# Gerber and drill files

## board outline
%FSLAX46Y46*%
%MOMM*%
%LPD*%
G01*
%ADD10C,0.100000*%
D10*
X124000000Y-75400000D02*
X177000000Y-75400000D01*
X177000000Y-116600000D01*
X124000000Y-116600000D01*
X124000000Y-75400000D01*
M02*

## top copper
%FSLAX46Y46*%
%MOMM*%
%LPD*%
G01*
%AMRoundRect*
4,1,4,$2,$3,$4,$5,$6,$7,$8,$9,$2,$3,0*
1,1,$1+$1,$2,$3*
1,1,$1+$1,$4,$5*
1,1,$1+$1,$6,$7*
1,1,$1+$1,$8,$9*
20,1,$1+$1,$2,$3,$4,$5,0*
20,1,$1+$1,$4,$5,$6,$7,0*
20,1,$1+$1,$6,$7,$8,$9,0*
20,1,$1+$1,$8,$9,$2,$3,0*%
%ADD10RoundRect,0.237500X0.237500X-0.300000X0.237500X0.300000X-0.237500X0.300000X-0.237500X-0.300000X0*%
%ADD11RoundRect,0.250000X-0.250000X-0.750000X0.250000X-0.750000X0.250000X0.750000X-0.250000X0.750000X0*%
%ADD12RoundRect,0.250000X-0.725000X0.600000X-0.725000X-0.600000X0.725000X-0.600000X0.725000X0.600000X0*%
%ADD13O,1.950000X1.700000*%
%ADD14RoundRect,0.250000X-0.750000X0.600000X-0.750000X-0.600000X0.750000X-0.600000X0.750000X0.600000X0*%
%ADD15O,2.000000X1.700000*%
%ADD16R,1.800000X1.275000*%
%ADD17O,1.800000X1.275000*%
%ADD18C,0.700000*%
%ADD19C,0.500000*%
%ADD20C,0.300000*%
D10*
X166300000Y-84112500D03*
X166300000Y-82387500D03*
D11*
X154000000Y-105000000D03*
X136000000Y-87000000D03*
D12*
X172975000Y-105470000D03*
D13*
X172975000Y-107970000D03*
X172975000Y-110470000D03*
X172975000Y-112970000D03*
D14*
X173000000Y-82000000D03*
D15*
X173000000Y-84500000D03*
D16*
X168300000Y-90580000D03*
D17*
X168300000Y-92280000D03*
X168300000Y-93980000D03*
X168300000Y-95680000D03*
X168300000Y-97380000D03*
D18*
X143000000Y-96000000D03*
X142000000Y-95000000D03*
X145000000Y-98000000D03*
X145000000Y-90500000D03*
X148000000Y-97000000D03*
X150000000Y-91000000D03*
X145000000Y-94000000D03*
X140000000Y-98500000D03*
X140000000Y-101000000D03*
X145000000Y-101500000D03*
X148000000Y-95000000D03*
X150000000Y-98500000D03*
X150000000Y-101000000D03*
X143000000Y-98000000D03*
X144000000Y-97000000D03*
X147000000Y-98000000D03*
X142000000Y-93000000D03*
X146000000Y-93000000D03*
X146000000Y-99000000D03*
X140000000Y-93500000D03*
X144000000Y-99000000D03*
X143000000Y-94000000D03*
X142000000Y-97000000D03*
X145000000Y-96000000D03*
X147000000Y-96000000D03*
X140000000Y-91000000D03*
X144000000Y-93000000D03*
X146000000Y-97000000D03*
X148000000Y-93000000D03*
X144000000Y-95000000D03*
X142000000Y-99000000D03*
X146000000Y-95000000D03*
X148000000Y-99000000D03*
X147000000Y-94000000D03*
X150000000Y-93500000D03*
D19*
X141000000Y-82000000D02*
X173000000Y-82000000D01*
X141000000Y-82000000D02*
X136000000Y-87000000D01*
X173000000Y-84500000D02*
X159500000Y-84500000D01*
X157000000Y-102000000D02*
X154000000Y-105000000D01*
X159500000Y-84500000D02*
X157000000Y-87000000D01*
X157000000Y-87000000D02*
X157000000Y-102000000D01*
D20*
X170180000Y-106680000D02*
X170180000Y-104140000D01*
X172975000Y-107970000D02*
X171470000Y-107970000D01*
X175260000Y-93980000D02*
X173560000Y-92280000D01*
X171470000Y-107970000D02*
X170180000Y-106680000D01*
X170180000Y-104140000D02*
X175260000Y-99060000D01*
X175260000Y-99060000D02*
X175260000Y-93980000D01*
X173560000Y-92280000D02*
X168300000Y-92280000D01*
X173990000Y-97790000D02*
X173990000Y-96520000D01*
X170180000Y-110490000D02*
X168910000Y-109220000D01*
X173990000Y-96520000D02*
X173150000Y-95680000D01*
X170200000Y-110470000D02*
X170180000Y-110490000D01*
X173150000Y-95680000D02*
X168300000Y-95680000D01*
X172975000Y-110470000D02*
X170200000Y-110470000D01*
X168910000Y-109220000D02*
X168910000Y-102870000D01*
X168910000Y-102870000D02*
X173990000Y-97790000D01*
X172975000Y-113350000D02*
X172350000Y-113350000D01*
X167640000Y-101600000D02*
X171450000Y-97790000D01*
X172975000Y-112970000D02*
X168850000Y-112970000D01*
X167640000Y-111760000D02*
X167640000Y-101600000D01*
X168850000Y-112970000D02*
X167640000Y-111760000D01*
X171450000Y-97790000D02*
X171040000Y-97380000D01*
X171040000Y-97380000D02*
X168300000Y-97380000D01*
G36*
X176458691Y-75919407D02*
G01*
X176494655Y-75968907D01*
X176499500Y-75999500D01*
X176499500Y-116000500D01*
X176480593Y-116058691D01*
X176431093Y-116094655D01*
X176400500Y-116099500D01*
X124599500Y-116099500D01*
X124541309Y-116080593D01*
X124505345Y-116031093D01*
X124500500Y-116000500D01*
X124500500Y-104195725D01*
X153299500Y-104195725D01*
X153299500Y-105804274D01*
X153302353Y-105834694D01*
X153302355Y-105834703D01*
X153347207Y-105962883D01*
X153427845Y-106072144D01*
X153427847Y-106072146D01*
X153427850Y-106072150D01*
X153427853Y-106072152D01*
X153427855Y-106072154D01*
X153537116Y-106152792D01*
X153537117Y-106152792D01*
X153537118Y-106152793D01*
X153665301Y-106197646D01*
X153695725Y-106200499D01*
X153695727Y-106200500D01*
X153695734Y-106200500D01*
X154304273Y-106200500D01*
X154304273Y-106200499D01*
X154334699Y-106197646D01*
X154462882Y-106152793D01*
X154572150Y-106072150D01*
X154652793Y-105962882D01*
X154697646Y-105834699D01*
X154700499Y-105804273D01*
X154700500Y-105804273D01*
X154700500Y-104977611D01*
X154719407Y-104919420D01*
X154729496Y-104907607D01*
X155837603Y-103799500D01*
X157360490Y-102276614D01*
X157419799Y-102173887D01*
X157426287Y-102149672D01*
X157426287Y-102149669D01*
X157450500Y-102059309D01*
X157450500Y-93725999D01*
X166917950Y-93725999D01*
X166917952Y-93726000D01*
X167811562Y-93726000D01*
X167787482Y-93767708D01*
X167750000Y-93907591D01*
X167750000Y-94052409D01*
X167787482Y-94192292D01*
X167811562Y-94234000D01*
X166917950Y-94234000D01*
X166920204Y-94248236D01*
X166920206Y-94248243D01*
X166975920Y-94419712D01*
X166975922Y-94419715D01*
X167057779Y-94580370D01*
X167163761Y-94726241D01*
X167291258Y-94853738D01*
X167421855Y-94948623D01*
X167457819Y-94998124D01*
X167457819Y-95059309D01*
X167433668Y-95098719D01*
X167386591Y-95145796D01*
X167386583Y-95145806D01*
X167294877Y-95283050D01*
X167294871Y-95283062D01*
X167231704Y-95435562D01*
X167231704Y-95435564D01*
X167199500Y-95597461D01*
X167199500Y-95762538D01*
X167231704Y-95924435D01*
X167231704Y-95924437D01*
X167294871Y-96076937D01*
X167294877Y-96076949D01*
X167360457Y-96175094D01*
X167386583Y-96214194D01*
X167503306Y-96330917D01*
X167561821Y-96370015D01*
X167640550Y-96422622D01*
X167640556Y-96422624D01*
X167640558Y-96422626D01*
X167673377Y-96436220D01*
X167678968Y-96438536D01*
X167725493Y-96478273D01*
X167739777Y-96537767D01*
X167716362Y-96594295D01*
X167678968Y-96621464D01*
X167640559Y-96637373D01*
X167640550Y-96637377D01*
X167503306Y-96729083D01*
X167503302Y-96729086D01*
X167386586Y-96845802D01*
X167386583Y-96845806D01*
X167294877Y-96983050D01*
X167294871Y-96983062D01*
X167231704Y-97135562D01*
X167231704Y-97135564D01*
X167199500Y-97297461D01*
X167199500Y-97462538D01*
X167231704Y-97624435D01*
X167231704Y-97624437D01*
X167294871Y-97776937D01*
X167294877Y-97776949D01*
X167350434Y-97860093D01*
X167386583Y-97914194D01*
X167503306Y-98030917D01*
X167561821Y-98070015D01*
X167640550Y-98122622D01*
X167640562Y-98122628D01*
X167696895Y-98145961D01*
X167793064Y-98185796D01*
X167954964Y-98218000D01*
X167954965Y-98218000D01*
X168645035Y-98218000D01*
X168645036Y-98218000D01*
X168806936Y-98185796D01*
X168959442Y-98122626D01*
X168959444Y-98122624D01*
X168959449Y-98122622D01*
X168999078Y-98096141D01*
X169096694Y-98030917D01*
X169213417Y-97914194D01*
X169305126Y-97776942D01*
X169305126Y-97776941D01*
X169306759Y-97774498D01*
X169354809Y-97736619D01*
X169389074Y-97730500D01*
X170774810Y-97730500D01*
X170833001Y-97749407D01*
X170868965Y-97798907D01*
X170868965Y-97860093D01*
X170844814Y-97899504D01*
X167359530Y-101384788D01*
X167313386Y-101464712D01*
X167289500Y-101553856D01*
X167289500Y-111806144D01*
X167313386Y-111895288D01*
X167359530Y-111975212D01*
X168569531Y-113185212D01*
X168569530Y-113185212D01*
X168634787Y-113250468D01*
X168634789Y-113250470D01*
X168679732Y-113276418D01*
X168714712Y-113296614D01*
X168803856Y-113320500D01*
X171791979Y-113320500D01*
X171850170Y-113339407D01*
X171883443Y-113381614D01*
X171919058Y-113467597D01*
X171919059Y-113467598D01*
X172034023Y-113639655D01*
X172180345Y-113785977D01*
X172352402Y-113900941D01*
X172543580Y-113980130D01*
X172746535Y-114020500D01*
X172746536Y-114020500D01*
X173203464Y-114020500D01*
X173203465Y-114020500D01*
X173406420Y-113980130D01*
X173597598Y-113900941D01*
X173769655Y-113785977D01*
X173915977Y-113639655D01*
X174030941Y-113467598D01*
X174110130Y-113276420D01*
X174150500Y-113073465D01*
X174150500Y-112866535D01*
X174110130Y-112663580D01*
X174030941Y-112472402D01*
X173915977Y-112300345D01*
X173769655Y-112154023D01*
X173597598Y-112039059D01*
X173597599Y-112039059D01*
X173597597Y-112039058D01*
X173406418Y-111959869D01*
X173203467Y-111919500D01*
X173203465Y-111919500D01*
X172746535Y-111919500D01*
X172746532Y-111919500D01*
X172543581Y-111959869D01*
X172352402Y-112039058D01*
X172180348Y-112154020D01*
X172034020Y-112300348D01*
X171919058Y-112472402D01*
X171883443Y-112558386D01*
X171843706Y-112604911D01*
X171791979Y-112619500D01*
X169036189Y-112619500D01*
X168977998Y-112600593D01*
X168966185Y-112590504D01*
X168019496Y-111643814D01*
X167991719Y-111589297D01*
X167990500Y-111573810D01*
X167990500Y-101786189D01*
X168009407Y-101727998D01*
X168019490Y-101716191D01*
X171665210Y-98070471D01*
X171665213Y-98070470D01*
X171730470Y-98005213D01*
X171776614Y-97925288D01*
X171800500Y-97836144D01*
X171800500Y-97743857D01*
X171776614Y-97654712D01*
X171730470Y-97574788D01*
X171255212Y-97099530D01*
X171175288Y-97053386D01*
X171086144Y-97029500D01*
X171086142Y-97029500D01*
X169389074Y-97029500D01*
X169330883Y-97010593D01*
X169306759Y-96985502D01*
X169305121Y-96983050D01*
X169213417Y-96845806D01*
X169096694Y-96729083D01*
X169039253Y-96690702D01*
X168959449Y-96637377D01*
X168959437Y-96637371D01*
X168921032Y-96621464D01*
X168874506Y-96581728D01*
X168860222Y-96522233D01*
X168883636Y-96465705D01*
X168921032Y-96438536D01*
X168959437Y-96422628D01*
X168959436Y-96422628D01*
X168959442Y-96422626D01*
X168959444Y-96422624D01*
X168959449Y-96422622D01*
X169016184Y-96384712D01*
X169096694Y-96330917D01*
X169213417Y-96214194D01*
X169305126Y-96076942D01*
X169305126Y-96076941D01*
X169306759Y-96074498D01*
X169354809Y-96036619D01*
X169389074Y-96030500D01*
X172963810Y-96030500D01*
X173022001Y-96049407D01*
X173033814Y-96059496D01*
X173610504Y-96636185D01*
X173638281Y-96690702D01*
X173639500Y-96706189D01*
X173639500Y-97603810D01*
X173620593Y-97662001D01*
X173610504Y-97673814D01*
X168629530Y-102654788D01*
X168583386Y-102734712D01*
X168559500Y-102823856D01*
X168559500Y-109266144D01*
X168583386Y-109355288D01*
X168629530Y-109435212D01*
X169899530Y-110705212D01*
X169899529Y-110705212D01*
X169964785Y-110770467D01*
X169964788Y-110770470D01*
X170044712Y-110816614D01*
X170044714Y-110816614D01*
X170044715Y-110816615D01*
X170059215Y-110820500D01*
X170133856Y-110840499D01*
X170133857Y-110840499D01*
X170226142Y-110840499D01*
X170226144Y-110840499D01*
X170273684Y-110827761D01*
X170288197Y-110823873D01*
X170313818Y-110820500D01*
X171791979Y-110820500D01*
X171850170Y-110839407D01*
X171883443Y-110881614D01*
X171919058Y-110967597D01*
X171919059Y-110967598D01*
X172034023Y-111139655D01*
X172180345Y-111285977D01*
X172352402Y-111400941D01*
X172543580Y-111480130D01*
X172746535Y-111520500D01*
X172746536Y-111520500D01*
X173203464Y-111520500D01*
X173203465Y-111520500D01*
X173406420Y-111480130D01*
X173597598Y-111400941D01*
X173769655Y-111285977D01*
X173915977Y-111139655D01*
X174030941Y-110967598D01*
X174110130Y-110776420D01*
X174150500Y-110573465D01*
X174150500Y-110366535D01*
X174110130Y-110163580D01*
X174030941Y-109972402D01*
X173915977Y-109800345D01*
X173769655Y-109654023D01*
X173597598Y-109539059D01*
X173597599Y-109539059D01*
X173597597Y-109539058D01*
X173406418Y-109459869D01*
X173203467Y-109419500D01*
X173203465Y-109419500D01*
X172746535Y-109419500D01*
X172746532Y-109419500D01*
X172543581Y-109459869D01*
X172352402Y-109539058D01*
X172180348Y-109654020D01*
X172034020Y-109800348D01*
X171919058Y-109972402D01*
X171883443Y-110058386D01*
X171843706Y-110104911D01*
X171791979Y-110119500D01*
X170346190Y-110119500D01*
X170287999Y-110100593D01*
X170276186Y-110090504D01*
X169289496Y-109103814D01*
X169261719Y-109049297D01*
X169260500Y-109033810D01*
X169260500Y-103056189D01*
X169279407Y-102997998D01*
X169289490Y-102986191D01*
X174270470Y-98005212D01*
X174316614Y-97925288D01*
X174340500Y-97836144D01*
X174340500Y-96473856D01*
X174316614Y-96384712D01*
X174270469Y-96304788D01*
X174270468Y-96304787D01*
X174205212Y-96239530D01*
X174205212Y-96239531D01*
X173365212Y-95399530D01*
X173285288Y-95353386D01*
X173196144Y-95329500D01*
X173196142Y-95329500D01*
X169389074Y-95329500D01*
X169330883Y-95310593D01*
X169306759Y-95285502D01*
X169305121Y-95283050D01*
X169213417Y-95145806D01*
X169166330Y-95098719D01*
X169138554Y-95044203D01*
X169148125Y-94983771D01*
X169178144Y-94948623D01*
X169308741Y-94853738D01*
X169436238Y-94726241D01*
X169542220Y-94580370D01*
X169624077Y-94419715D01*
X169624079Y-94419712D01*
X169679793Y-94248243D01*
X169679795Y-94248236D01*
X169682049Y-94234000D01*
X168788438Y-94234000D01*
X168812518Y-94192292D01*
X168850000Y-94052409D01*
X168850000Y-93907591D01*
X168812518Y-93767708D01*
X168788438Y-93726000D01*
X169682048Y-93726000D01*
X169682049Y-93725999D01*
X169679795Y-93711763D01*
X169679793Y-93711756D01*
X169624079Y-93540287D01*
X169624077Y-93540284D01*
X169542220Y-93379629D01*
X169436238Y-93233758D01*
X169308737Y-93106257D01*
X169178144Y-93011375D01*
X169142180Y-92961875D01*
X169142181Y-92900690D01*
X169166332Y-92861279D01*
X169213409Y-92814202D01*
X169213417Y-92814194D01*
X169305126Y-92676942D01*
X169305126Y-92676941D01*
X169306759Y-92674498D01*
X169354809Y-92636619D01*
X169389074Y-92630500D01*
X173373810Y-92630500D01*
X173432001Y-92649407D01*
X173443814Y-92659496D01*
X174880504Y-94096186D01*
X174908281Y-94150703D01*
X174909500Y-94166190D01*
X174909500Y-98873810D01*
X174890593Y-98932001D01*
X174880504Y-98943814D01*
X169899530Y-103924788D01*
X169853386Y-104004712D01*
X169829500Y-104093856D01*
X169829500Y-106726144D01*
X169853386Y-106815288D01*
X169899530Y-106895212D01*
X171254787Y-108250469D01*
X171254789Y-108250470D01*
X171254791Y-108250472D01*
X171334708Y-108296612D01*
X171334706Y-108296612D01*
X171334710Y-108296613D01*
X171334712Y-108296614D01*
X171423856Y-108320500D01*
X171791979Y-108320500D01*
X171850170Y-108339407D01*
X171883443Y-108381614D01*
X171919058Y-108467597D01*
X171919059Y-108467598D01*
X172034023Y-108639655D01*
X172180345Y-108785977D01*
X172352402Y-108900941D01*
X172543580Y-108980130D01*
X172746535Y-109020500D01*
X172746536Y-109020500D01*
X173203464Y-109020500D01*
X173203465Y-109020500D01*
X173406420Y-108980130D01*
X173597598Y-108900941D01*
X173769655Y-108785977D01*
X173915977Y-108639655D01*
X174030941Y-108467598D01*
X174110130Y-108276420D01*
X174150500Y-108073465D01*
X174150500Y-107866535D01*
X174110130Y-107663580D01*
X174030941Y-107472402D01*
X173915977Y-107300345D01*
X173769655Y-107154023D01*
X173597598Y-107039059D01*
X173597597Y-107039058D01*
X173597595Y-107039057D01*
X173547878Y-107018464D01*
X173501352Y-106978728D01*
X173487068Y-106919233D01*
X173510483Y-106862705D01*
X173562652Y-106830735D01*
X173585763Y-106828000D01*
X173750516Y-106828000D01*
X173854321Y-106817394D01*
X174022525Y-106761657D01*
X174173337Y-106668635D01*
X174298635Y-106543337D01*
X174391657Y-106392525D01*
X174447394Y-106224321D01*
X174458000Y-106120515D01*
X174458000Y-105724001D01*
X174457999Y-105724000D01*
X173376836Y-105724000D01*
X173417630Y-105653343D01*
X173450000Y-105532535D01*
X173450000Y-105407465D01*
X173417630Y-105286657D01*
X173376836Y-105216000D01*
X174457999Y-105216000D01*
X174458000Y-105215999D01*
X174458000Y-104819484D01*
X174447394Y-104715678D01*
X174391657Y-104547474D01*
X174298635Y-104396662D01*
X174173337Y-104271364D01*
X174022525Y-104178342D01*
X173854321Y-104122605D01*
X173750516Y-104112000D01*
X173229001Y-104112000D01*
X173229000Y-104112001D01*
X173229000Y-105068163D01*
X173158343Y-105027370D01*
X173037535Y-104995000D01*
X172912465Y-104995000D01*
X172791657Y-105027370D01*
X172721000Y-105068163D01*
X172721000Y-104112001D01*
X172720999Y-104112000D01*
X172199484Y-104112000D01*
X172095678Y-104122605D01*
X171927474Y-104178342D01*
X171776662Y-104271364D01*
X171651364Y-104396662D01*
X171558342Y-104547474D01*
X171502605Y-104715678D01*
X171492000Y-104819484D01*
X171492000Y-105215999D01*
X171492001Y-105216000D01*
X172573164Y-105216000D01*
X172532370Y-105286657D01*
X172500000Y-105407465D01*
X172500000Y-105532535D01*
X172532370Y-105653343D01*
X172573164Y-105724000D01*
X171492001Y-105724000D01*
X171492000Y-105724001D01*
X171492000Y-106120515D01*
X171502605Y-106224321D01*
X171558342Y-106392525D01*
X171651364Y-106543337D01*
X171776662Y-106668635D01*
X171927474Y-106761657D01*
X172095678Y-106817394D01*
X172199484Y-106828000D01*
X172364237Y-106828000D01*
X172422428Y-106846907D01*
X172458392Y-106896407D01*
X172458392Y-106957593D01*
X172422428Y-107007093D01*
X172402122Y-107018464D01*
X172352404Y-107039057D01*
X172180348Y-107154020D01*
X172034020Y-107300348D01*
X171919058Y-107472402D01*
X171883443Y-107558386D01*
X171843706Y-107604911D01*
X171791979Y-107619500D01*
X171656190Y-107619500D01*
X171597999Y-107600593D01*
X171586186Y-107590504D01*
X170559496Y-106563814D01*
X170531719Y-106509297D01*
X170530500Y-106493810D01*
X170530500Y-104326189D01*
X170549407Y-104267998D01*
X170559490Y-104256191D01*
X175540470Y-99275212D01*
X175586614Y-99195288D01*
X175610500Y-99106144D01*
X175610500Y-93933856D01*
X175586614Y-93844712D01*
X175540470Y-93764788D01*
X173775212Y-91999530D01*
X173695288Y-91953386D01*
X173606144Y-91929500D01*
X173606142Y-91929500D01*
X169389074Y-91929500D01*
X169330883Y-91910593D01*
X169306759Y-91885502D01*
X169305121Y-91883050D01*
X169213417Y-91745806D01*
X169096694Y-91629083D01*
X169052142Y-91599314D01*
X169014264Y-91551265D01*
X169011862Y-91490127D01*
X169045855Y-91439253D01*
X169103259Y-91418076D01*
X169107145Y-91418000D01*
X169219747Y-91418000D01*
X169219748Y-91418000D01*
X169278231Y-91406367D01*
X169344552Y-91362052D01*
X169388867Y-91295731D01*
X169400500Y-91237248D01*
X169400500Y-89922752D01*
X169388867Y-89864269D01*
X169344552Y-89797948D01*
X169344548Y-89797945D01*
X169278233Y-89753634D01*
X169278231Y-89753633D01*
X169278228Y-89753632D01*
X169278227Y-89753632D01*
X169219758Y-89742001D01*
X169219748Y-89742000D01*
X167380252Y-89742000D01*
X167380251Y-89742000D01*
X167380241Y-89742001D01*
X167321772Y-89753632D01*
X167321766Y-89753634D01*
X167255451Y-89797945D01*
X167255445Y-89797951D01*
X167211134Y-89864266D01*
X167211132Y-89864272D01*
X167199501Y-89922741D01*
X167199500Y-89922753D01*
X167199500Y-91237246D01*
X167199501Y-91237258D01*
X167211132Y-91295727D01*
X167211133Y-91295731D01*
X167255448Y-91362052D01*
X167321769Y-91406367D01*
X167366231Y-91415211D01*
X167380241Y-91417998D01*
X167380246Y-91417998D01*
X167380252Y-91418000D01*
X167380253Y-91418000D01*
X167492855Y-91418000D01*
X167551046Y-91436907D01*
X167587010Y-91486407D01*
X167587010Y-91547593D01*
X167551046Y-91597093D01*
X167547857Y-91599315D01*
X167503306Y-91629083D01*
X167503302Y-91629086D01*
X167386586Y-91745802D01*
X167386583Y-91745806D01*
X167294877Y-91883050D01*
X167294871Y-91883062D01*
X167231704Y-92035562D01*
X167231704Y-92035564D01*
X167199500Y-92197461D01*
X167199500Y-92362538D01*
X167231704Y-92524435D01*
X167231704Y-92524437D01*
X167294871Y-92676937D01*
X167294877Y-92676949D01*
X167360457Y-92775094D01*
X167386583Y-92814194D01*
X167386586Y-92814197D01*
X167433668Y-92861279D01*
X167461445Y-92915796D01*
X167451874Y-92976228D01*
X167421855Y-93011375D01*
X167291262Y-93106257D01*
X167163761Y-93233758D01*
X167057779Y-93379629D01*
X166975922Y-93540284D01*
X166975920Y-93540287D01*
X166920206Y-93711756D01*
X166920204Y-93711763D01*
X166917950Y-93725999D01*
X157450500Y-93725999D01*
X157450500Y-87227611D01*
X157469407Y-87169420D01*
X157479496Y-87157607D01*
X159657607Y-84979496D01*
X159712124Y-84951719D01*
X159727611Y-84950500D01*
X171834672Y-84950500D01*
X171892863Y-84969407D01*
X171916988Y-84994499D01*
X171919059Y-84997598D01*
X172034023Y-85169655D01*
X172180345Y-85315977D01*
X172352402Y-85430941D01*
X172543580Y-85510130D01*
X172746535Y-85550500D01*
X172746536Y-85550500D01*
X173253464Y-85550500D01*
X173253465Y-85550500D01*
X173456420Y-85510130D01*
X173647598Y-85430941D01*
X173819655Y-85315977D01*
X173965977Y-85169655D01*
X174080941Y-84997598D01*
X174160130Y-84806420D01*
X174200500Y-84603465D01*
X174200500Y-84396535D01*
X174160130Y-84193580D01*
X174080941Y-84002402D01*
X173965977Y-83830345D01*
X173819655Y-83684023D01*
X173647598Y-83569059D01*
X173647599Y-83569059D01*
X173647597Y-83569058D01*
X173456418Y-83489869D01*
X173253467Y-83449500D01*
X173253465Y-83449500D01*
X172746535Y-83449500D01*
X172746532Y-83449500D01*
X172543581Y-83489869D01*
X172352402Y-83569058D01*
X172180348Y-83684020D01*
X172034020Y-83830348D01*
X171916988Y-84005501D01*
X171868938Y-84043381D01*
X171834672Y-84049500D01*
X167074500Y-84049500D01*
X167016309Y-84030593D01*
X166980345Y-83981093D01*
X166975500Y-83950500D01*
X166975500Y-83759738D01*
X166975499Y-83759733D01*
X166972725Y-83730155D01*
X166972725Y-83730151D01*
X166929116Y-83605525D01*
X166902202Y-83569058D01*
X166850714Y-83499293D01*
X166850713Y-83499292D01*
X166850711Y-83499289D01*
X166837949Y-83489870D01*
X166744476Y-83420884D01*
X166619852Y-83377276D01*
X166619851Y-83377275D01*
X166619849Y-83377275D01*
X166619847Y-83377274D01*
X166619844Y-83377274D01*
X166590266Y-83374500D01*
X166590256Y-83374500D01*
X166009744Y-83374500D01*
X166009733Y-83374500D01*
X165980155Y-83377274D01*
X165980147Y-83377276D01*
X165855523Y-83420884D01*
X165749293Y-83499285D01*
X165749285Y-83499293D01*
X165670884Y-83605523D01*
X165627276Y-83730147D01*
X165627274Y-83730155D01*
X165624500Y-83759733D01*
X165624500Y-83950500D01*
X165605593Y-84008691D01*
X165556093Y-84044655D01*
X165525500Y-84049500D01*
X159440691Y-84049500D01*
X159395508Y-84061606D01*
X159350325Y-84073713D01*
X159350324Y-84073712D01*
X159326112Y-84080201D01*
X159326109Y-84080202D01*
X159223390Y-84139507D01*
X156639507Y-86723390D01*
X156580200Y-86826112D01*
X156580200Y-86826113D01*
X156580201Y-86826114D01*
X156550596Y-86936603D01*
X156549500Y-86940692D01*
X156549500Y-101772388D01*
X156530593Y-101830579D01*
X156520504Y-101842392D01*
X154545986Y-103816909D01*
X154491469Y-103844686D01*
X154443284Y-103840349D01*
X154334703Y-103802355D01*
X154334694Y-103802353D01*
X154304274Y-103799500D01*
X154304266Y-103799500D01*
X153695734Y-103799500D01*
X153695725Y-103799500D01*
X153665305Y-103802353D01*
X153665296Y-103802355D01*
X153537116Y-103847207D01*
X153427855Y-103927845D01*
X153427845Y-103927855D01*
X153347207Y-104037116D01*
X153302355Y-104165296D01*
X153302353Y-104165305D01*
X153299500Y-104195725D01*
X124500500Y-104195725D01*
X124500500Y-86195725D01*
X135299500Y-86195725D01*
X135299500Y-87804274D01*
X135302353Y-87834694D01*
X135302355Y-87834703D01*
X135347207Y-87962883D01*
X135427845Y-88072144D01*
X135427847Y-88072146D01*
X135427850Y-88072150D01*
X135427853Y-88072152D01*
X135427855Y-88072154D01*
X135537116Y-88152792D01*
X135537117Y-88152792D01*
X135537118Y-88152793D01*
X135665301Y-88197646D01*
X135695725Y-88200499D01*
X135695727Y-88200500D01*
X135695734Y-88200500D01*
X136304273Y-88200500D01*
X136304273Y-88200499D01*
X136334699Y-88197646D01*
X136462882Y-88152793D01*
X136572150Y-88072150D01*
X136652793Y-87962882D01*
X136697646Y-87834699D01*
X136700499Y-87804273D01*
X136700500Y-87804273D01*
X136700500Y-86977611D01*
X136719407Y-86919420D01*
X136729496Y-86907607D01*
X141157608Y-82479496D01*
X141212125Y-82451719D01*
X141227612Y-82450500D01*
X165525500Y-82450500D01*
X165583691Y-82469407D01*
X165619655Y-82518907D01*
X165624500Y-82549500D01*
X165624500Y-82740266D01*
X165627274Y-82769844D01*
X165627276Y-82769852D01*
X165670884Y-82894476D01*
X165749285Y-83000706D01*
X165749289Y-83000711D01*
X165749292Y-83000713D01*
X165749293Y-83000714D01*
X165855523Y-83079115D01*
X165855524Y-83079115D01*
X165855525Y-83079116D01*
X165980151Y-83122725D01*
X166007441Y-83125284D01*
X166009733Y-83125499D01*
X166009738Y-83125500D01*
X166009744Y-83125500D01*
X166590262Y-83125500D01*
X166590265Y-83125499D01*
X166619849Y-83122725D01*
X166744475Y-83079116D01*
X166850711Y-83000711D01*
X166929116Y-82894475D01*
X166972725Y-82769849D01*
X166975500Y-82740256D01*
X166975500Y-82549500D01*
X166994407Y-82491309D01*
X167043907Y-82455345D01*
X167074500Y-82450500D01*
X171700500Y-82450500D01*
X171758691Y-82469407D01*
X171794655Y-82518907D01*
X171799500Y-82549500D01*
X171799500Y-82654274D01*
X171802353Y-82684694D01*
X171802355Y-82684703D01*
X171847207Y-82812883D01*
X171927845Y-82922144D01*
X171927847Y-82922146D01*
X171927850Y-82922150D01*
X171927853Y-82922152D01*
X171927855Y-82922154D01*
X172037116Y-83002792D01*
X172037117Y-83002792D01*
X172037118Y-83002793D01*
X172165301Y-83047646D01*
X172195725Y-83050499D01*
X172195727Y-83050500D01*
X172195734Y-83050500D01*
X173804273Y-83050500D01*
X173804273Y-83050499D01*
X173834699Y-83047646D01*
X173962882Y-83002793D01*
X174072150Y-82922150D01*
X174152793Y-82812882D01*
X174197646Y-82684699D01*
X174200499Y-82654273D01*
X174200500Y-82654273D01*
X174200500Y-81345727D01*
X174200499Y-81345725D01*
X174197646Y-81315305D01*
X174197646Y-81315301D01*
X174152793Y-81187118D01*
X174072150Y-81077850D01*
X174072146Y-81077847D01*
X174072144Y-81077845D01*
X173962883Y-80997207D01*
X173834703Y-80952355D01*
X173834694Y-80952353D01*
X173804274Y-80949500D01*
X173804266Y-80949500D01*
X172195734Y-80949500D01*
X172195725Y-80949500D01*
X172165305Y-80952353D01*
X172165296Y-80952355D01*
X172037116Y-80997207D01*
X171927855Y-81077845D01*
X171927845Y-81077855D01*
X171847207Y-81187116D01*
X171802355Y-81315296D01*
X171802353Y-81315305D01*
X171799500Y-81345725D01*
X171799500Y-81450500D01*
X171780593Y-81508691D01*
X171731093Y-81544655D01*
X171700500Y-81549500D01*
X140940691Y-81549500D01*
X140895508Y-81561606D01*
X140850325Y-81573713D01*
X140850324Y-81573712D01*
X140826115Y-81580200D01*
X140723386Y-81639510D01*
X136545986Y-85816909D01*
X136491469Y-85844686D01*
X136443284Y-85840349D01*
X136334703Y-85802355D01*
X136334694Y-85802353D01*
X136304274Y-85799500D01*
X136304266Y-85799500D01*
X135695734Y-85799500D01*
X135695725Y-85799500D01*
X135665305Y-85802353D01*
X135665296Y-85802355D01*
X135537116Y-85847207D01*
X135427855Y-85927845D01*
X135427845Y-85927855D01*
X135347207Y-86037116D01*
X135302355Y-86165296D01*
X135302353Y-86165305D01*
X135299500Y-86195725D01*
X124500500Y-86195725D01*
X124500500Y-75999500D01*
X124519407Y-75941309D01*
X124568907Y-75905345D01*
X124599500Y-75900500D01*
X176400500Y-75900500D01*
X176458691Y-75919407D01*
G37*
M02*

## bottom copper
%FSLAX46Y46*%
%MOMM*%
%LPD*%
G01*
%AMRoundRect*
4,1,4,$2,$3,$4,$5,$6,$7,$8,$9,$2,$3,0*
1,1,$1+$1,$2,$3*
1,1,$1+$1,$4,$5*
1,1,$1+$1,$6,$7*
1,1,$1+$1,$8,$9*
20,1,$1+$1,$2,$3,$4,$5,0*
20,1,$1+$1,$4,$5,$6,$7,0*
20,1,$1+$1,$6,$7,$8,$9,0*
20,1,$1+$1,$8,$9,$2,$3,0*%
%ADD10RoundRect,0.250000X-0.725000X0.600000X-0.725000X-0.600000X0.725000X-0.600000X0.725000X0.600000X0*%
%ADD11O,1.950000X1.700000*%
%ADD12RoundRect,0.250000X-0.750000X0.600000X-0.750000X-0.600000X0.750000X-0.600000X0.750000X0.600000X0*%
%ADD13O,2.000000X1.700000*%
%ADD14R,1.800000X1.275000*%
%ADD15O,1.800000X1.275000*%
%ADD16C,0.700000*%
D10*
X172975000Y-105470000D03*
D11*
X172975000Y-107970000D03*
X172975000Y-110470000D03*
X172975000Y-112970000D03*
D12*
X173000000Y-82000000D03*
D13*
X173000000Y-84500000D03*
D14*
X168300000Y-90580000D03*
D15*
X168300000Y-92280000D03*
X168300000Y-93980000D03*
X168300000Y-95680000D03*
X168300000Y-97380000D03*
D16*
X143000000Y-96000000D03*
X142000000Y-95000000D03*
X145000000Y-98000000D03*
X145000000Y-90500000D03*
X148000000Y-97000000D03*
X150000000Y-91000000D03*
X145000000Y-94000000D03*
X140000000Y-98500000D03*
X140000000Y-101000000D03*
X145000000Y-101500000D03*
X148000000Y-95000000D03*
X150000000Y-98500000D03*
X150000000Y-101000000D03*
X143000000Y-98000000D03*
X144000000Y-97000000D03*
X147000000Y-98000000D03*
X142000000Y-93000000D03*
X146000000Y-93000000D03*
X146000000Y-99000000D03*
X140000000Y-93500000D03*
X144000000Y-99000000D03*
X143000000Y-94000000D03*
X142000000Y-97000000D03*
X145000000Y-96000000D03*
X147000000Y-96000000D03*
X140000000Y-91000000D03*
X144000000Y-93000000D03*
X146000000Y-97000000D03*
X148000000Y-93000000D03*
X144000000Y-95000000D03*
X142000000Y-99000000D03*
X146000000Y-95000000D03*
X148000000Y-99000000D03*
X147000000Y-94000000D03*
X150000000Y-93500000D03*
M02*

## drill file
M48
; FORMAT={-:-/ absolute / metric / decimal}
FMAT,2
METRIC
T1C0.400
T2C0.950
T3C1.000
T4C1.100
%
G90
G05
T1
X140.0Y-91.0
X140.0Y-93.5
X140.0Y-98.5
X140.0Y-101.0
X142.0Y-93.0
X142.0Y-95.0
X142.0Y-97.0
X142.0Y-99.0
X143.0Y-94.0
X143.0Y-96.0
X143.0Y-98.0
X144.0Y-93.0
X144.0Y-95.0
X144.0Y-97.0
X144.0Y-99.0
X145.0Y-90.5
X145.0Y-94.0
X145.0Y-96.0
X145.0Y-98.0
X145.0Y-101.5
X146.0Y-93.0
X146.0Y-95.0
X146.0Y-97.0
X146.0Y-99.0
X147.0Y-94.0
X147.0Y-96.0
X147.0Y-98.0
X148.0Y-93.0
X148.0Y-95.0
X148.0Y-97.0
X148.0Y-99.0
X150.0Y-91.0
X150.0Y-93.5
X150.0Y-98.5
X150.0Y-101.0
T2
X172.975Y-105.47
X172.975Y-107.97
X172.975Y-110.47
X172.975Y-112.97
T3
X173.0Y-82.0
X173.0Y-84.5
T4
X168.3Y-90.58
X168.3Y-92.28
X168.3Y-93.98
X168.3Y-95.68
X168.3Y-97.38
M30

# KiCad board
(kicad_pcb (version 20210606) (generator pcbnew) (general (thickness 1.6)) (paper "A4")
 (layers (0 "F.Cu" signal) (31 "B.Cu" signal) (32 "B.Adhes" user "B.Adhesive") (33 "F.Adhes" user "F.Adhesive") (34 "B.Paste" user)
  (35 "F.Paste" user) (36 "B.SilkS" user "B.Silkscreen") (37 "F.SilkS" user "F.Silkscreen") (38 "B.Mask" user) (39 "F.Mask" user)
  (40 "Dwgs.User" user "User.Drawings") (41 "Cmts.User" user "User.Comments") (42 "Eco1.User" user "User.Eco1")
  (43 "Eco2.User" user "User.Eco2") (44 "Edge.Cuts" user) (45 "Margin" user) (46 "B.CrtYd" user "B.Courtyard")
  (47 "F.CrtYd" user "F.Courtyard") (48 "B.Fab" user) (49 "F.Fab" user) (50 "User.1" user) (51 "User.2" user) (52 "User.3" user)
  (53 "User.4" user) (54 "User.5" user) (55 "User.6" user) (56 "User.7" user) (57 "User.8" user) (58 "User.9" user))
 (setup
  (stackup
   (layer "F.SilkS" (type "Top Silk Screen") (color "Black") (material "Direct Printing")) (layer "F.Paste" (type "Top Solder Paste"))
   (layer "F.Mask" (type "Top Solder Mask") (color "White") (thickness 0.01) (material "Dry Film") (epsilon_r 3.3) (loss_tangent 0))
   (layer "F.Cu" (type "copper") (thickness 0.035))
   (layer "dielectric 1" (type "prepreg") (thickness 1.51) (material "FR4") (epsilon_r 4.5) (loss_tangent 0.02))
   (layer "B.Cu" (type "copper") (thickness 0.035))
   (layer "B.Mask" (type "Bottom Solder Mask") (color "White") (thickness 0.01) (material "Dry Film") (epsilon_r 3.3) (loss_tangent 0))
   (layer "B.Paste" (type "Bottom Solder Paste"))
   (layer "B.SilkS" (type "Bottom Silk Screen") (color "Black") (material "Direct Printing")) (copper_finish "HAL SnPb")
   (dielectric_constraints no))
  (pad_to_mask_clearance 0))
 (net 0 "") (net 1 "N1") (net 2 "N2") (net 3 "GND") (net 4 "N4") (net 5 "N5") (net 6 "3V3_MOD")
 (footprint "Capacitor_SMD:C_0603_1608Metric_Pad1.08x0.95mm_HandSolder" (layer "F.Cu") (at 166.3 83.25 90)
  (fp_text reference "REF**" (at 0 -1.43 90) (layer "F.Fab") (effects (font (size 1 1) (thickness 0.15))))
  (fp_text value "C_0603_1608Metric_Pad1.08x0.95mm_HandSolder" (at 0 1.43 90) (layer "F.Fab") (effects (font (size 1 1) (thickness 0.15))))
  (pad "1" smd roundrect locked (at -0.8625 0 90) (size 1.075 0.95) (layers "F.Cu" "F.Paste" "F.Mask") (roundrect_rratio 0.25) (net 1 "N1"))
  (pad "2" smd roundrect locked (at 0.8625 0 90) (size 1.075 0.95) (layers "F.Cu" "F.Paste" "F.Mask") (roundrect_rratio 0.25) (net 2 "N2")))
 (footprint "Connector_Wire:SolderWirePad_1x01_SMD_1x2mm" (layer "F.Cu") (at 154 105)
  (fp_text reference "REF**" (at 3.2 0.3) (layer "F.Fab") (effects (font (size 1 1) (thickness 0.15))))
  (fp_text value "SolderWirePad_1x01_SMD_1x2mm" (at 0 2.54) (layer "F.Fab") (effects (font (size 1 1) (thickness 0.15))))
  (pad "1" smd roundrect locked (at 0 0) (size 1 2) (layers "F.Cu" "F.Paste" "F.Mask") (roundrect_rratio 0.25) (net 1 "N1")))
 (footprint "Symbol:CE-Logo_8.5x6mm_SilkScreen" (layer "F.Cu") (at 139.18419 112.268)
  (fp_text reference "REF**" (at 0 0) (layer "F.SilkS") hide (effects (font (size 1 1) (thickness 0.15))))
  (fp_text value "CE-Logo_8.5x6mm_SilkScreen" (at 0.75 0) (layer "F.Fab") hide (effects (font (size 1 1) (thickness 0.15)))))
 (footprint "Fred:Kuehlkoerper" (layer "F.Cu") (at 144.66 95.96)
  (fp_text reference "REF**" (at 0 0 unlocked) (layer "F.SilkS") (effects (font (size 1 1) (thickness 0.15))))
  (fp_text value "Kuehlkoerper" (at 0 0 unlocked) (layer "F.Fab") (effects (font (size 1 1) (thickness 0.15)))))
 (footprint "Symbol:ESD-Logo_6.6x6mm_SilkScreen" (layer "F.Cu") (at 129.18419 112.268)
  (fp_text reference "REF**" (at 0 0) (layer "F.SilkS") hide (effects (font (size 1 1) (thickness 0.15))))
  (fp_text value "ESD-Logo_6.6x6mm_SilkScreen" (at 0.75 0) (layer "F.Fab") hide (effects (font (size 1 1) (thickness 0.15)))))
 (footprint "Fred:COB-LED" (layer "F.Cu") (at 144.81 95.85)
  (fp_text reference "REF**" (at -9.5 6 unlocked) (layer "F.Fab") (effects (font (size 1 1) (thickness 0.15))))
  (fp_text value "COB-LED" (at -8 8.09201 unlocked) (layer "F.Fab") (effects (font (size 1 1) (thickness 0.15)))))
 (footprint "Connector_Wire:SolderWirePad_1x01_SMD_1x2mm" (layer "F.Cu") (at 136 87)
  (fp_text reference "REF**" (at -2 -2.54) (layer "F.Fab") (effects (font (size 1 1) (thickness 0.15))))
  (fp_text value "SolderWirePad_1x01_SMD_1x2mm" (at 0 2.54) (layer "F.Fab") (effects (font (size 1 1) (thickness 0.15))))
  (pad "1" smd roundrect locked (at 0 0) (size 1 2) (layers "F.Cu" "F.Paste" "F.Mask") (roundrect_rratio 0.25) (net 2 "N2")))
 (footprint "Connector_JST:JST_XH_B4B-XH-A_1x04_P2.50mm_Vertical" (layer "B.Cu") (at 172.975 105.47 -90)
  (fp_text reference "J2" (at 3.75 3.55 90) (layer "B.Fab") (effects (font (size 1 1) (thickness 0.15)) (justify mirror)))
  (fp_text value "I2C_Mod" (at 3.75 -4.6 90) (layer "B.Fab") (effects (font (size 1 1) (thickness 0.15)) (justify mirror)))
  (pad "1" thru_hole roundrect locked (at 0 0 270) (size 1.7 1.95) (drill 0.95) (layers *.Cu *.Mask) (roundrect_rratio 0.1470588235)
   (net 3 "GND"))
  (pad "2" thru_hole oval locked (at 2.5 0 270) (size 1.7 1.95) (drill 0.95) (layers *.Cu *.Mask) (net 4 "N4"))
  (pad "3" thru_hole oval locked (at 5 0 270) (size 1.7 1.95) (drill 0.95) (layers *.Cu *.Mask) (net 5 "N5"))
  (pad "4" thru_hole oval locked (at 7.5 0 270) (size 1.7 1.95) (drill 0.95) (layers *.Cu *.Mask) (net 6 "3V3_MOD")))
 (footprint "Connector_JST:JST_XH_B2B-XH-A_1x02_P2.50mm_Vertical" (layer "B.Cu") (at 173 82 -90)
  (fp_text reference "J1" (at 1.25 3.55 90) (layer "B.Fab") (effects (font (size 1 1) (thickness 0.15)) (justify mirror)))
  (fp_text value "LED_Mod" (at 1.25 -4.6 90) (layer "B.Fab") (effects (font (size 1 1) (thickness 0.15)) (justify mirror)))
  (pad "1" thru_hole roundrect locked (at 0 0 270) (size 1.7 2) (drill 1) (layers *.Cu *.Mask) (roundrect_rratio 0.1470588235) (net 2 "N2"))
  (pad "2" thru_hole oval locked (at 2.5 0 270) (size 1.7 2) (drill 1) (layers *.Cu *.Mask) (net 1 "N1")))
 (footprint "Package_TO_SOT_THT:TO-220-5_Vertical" (layer "B.Cu") (at 168.3 90.58 -90)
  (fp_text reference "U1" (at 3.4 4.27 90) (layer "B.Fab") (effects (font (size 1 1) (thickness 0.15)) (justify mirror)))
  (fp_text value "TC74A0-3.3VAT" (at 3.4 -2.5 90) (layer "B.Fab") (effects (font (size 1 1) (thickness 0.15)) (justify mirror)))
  (pad "1" thru_hole rect locked (at 0 0 270) (size 1.275 1.8) (drill 1.1) (layers *.Cu *.Mask))
  (pad "2" thru_hole oval locked (at 1.7 0 270) (size 1.275 1.8) (drill 1.1) (layers *.Cu *.Mask) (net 4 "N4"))
  (pad "3" thru_hole oval locked (at 3.4 0 270) (size 1.275 1.8) (drill 1.1) (layers *.Cu *.Mask) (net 3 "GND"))
  (pad "4" thru_hole oval locked (at 5.1 0 270) (size 1.275 1.8) (drill 1.1) (layers *.Cu *.Mask) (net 5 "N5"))
  (pad "5" thru_hole oval locked (at 6.8 0 270) (size 1.275 1.8) (drill 1.1) (layers *.Cu *.Mask) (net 6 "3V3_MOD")))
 (gr_rect (start 177 116.6) (end 124 75.4) (layer "Edge.Cuts") (width 0.1) (fill none))
 (segment (start 141 82) (end 173 82) (width 0.5) (layer "F.Cu") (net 2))
 (segment (start 141 82) (end 136 87) (width 0.5) (layer "F.Cu") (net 2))
 (segment (start 173 84.5) (end 159.5 84.5) (width 0.5) (layer "F.Cu") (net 1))
 (segment (start 157 102) (end 154 105) (width 0.5) (layer "F.Cu") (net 1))
 (segment (start 159.5 84.5) (end 157 87) (width 0.5) (layer "F.Cu") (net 1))
 (segment (start 157 87) (end 157 102) (width 0.5) (layer "F.Cu") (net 1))
 (via (at 143 96) (size 0.7) (drill 0.4) (layers "F.Cu" "B.Cu") (free) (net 3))
 (via (at 142 95) (size 0.7) (drill 0.4) (layers "F.Cu" "B.Cu") (free) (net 3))
 (via (at 145 98) (size 0.7) (drill 0.4) (layers "F.Cu" "B.Cu") (free) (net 3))
 (via (at 145 90.5) (size 0.7) (drill 0.4) (layers "F.Cu" "B.Cu") (free) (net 3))
 (via (at 148 97) (size 0.7) (drill 0.4) (layers "F.Cu" "B.Cu") (free) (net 3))
 (via (at 150 91) (size 0.7) (drill 0.4) (layers "F.Cu" "B.Cu") (free) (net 3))
 (via (at 145 94) (size 0.7) (drill 0.4) (layers "F.Cu" "B.Cu") (free) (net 3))
 (via (at 140 98.5) (size 0.7) (drill 0.4) (layers "F.Cu" "B.Cu") (free) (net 3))
 (via (at 140 101) (size 0.7) (drill 0.4) (layers "F.Cu" "B.Cu") (free) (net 3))
 (via (at 145 101.5) (size 0.7) (drill 0.4) (layers "F.Cu" "B.Cu") (free) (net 3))
 (via (at 148 95) (size 0.7) (drill 0.4) (layers "F.Cu" "B.Cu") (free) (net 3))
 (via (at 150 98.5) (size 0.7) (drill 0.4) (layers "F.Cu" "B.Cu") (free) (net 3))
 (via (at 150 101) (size 0.7) (drill 0.4) (layers "F.Cu" "B.Cu") (free) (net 3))
 (via (at 143 98) (size 0.7) (drill 0.4) (layers "F.Cu" "B.Cu") (free) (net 3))
 (via (at 144 97) (size 0.7) (drill 0.4) (layers "F.Cu" "B.Cu") (free) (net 3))
 (via (at 147 98) (size 0.7) (drill 0.4) (layers "F.Cu" "B.Cu") (free) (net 3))
 (via (at 142 93) (size 0.7) (drill 0.4) (layers "F.Cu" "B.Cu") (free) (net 3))
 (via (at 146 93) (size 0.7) (drill 0.4) (layers "F.Cu" "B.Cu") (free) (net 3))
 (via (at 146 99) (size 0.7) (drill 0.4) (layers "F.Cu" "B.Cu") (free) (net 3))
 (via (at 140 93.5) (size 0.7) (drill 0.4) (layers "F.Cu" "B.Cu") (free) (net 3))
 (via (at 144 99) (size 0.7) (drill 0.4) (layers "F.Cu" "B.Cu") (free) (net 3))
 (via (at 143 94) (size 0.7) (drill 0.4) (layers "F.Cu" "B.Cu") (free) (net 3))
 (via (at 142 97) (size 0.7) (drill 0.4) (layers "F.Cu" "B.Cu") (free) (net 3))
 (via (at 145 96) (size 0.7) (drill 0.4) (layers "F.Cu" "B.Cu") (free) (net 3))
 (via (at 147 96) (size 0.7) (drill 0.4) (layers "F.Cu" "B.Cu") (free) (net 3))
 (via (at 140 91) (size 0.7) (drill 0.4) (layers "F.Cu" "B.Cu") (free) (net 3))
 (via (at 144 93) (size 0.7) (drill 0.4) (layers "F.Cu" "B.Cu") (free) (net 3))
 (via (at 146 97) (size 0.7) (drill 0.4) (layers "F.Cu" "B.Cu") (free) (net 3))
 (via (at 148 93) (size 0.7) (drill 0.4) (layers "F.Cu" "B.Cu") (free) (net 3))
 (via (at 144 95) (size 0.7) (drill 0.4) (layers "F.Cu" "B.Cu") (free) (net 3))
 (via (at 142 99) (size 0.7) (drill 0.4) (layers "F.Cu" "B.Cu") (free) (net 3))
 (via (at 146 95) (size 0.7) (drill 0.4) (layers "F.Cu" "B.Cu") (free) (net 3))
 (via (at 148 99) (size 0.7) (drill 0.4) (layers "F.Cu" "B.Cu") (free) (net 3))
 (via (at 147 94) (size 0.7) (drill 0.4) (layers "F.Cu" "B.Cu") (free) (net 3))
 (via (at 150 93.5) (size 0.7) (drill 0.4) (layers "F.Cu" "B.Cu") (free) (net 3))
 (segment (start 170.18 106.68) (end 170.18 104.14) (width 0.3) (layer "F.Cu") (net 4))
 (segment (start 172.975 107.97) (end 171.47 107.97) (width 0.3) (layer "F.Cu") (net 4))
 (segment (start 175.26 93.98) (end 173.56 92.28) (width 0.3) (layer "F.Cu") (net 4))
 (segment (start 171.47 107.97) (end 170.18 106.68) (width 0.3) (layer "F.Cu") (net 4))
 (segment (start 170.18 104.14) (end 175.26 99.06) (width 0.3) (layer "F.Cu") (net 4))
 (segment (start 175.26 99.06) (end 175.26 93.98) (width 0.3) (layer "F.Cu") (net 4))
 (segment (start 173.56 92.28) (end 168.3 92.28) (width 0.3) (layer "F.Cu") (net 4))
 (segment (start 173.99 97.79) (end 173.99 96.52) (width 0.3) (layer "F.Cu") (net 5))
 (segment (start 170.18 110.49) (end 168.91 109.22) (width 0.3) (layer "F.Cu") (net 5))
 (segment (start 173.99 96.52) (end 173.15 95.68) (width 0.3) (layer "F.Cu") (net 5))
 (segment (start 170.2 110.47) (end 170.18 110.49) (width 0.3) (layer "F.Cu") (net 5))
 (segment (start 173.15 95.68) (end 168.3 95.68) (width 0.3) (layer "F.Cu") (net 5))
 (segment (start 172.975 110.47) (end 170.2 110.47) (width 0.3) (layer "F.Cu") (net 5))
 (segment (start 168.91 109.22) (end 168.91 102.87) (width 0.3) (layer "F.Cu") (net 5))
 (segment (start 168.91 102.87) (end 173.99 97.79) (width 0.3) (layer "F.Cu") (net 5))
 (segment (start 172.975 113.35) (end 172.35 113.35) (width 0.3) (layer "F.Cu") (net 6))
 (segment (start 167.64 101.6) (end 171.45 97.79) (width 0.3) (layer "F.Cu") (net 6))
 (segment (start 172.975 112.97) (end 168.85 112.97) (width 0.3) (layer "F.Cu") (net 6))
 (segment (start 167.64 111.76) (end 167.64 101.6) (width 0.3) (layer "F.Cu") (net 6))
 (segment (start 168.85 112.97) (end 167.64 111.76) (width 0.3) (layer "F.Cu") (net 6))
 (segment (start 171.45 97.79) (end 171.04 97.38) (width 0.3) (layer "F.Cu") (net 6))
 (segment (start 171.04 97.38) (end 168.3 97.38) (width 0.3) (layer "F.Cu") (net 6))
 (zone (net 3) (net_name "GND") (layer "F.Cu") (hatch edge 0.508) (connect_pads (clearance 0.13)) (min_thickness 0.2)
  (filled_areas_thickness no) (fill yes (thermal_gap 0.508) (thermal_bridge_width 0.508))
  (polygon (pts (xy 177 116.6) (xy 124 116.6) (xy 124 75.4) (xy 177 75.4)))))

